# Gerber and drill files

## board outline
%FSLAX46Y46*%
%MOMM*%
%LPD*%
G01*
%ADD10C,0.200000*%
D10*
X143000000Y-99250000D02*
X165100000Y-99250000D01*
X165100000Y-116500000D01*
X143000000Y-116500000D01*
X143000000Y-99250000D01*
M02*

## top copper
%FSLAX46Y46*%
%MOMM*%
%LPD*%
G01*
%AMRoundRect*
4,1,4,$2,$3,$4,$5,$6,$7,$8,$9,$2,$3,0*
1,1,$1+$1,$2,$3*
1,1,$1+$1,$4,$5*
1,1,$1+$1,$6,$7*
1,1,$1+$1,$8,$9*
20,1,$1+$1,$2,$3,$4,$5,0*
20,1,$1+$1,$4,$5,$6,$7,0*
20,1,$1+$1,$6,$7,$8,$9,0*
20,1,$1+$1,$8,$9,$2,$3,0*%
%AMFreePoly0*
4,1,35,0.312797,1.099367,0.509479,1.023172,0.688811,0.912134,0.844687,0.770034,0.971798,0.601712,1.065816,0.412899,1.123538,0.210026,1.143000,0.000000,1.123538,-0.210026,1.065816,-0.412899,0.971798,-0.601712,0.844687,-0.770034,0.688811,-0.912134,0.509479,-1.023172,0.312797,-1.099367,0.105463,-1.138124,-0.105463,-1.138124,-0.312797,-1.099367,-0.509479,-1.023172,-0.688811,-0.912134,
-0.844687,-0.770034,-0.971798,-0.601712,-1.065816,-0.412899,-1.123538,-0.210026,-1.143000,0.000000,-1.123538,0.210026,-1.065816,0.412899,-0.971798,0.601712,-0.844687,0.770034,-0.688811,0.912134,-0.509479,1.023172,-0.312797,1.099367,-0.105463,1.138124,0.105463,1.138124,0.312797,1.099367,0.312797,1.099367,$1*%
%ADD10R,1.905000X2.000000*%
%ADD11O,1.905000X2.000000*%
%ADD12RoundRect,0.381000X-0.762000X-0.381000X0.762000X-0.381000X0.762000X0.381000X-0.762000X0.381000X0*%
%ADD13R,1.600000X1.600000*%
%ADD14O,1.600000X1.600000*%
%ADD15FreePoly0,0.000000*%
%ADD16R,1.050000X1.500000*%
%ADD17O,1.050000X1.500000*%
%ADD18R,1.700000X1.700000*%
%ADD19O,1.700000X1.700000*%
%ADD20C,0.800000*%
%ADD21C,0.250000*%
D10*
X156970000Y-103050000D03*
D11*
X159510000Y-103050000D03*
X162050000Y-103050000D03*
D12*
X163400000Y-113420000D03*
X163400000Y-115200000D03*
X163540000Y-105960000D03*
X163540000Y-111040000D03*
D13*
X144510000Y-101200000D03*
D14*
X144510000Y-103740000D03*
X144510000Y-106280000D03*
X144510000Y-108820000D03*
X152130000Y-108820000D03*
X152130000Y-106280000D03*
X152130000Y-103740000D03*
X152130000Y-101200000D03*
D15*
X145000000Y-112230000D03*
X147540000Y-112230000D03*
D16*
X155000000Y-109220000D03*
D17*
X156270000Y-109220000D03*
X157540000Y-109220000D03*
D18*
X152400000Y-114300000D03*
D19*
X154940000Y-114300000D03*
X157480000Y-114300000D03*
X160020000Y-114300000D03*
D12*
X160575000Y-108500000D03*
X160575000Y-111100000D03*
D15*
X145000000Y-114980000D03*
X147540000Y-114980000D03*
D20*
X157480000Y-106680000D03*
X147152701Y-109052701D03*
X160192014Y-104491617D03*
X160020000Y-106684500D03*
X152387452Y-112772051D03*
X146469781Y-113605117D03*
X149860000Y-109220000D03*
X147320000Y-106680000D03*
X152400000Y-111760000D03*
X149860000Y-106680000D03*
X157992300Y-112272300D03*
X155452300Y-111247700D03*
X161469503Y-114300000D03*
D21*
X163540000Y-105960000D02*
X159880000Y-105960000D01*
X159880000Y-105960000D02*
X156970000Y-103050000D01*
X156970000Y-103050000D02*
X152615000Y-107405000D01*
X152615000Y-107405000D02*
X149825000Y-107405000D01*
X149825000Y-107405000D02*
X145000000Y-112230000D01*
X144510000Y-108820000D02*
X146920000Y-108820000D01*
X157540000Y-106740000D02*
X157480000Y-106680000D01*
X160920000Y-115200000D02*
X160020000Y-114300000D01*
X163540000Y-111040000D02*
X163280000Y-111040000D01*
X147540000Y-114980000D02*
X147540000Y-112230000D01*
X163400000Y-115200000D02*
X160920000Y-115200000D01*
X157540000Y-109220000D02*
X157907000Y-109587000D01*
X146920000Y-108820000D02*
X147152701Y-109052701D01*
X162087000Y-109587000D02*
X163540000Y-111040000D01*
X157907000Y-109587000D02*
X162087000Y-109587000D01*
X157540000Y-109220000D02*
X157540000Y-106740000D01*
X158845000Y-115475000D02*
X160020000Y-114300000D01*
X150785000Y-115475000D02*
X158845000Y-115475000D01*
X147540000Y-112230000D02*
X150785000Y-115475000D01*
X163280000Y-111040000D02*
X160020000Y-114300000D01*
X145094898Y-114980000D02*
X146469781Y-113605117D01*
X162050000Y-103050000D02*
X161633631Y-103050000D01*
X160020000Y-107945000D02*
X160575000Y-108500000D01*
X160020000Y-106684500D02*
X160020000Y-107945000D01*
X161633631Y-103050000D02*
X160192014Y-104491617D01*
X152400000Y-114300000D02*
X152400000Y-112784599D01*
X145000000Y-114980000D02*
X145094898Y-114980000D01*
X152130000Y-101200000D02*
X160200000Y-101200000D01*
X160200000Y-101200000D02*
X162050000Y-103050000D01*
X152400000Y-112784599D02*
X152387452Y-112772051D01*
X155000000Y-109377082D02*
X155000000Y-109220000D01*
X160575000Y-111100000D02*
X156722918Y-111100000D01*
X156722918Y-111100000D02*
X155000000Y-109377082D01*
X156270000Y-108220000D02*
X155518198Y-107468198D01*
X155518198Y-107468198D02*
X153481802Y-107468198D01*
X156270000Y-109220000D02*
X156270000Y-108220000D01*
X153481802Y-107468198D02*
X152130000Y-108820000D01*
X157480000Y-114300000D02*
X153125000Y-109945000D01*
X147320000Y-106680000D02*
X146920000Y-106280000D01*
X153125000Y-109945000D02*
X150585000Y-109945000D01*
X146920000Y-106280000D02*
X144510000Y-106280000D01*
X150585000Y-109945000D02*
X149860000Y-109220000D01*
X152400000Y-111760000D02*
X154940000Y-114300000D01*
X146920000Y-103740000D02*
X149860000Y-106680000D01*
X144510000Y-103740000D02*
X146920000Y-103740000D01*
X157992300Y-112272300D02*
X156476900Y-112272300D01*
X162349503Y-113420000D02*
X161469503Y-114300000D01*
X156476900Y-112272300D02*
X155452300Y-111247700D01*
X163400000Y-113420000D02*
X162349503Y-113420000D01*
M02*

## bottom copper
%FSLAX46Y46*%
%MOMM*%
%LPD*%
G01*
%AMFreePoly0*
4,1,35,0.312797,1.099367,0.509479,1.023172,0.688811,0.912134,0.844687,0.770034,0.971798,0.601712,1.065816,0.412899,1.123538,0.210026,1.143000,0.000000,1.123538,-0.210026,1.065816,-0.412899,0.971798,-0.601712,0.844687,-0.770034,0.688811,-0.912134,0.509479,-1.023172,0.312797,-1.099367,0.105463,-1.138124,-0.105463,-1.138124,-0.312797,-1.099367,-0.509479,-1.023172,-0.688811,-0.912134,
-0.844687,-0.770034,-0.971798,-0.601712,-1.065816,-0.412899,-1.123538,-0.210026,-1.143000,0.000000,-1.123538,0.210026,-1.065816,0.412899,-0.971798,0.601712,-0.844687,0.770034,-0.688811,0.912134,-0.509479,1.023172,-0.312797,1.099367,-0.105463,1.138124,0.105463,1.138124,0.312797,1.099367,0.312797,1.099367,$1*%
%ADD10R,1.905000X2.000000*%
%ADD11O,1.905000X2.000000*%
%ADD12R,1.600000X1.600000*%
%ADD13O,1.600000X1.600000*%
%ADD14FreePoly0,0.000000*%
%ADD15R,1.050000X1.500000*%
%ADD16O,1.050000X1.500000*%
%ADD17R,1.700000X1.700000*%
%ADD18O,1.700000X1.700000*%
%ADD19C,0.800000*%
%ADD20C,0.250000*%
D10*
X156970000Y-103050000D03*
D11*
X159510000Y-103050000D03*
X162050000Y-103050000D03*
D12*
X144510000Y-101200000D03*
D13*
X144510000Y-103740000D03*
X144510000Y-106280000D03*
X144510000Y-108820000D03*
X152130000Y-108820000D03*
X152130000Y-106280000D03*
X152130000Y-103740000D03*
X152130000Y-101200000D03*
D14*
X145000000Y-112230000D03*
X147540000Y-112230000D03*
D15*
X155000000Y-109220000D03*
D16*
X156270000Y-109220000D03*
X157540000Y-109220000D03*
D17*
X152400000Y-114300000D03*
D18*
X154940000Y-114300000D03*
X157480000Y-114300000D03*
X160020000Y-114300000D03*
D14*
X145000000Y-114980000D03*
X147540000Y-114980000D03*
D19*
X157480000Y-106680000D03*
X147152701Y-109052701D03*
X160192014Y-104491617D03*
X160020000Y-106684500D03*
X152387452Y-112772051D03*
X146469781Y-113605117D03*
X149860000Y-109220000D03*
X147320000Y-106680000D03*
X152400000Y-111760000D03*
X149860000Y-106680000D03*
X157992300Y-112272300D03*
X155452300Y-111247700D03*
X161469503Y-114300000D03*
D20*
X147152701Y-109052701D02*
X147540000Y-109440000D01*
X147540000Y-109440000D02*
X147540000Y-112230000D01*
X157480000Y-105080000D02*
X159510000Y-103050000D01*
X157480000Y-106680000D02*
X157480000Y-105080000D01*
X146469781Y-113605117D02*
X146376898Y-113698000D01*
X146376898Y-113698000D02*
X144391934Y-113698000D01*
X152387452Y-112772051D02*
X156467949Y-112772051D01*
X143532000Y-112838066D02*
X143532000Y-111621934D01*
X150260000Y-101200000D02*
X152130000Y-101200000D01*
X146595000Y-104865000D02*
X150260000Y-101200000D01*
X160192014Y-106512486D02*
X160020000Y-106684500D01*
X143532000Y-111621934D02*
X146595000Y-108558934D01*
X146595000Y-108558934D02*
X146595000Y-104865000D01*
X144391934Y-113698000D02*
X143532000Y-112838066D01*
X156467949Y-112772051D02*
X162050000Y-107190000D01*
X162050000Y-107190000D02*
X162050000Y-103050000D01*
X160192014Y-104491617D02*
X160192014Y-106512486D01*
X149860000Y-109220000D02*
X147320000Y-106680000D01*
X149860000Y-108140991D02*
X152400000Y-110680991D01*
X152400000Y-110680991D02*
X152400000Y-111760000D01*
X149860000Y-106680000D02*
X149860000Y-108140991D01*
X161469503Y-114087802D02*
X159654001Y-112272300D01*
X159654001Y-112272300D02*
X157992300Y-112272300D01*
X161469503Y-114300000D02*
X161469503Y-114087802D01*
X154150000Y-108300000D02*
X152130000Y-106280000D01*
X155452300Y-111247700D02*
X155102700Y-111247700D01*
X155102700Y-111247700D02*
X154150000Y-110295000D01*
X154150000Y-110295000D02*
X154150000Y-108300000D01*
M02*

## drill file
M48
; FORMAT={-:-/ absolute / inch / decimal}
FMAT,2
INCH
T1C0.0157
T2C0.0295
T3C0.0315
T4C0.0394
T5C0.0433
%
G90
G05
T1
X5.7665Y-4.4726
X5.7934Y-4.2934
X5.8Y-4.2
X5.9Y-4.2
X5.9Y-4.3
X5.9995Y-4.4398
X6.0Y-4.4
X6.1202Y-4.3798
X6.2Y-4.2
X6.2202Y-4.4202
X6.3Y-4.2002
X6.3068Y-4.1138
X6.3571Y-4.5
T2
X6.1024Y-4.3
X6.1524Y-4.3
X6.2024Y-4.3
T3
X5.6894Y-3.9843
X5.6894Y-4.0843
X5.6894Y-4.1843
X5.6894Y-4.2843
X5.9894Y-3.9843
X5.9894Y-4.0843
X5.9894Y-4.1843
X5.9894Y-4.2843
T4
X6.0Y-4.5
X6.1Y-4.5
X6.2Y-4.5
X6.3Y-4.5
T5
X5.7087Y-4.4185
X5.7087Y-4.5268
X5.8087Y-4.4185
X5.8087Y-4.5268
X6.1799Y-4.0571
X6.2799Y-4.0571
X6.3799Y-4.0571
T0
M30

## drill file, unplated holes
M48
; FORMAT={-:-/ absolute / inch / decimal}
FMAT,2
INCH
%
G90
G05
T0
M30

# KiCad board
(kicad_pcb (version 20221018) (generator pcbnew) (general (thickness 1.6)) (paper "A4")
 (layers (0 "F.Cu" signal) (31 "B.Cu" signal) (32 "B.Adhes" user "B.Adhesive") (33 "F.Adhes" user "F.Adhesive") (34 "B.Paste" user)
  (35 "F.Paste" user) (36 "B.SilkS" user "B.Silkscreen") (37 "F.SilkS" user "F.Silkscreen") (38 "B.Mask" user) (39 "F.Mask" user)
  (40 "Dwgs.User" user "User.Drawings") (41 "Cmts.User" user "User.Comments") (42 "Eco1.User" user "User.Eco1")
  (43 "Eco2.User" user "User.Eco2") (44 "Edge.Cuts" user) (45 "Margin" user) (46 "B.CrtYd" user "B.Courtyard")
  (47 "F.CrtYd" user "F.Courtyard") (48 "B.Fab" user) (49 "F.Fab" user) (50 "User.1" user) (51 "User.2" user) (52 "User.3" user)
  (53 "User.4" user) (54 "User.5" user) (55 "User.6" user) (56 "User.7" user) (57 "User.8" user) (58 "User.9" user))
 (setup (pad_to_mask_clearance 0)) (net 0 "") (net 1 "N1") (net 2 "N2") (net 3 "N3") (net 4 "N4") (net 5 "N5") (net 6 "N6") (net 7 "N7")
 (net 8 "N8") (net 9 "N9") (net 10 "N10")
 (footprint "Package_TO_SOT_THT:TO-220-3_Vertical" (layer "F.Cu") (at 156.97 103.05)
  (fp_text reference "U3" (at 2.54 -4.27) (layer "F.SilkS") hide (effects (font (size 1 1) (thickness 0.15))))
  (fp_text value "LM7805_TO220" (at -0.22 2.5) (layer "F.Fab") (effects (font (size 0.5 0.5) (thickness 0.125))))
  (pad "1" thru_hole rect (at 0 0) (size 1.905 2) (drill 1.1) (layers "*.Cu" "*.Mask") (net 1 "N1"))
  (pad "2" thru_hole oval (at 2.54 0) (size 1.905 2) (drill 1.1) (layers "*.Cu" "*.Mask") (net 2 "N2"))
  (pad "3" thru_hole oval (at 5.08 0) (size 1.905 2) (drill 1.1) (layers "*.Cu" "*.Mask") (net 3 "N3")))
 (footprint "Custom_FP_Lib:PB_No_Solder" (layer "F.Cu") (at 163.4 118.5)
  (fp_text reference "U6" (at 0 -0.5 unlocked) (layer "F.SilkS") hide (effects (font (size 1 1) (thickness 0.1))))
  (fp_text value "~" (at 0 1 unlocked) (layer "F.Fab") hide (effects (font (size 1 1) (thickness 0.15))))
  (pad "1" smd roundrect (at 0 -5.08) (size 2.286 1.524) (layers "F.Cu" "F.Paste" "F.Mask") (roundrect_rratio 0.25) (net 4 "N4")
   (thermal_bridge_angle 45))
  (pad "2" smd roundrect (at 0 -3.3) (size 2.286 1.524) (layers "F.Cu" "F.Paste" "F.Mask") (roundrect_rratio 0.25) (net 2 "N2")
   (thermal_bridge_angle 45)))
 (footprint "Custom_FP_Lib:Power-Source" (layer "F.Cu") (at 161 108.5)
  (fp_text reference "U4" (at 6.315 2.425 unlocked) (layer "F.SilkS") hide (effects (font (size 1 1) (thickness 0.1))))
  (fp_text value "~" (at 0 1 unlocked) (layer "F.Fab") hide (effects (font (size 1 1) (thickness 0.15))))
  (pad "1" smd roundrect (at 2.54 -2.54) (size 2.286 1.524) (layers "F.Cu" "F.Paste" "F.Mask") (roundrect_rratio 0.25) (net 1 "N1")
   (thermal_bridge_angle 45))
  (pad "2" smd roundrect (at 2.54 2.54) (size 2.286 1.524) (layers "F.Cu" "F.Paste" "F.Mask") (roundrect_rratio 0.25) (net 2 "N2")
   (thermal_bridge_angle 45)))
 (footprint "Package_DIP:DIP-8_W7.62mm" (layer "F.Cu") (at 144.51 101.2)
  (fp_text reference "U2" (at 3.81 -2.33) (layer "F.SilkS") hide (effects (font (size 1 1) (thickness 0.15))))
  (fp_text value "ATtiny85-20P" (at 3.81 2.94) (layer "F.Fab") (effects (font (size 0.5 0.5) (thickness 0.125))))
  (pad "1" thru_hole rect (at 0 0) (size 1.6 1.6) (drill 0.8) (layers "*.Cu" "*.Mask") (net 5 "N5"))
  (pad "2" thru_hole oval (at 0 2.54) (size 1.6 1.6) (drill 0.8) (layers "*.Cu" "*.Mask") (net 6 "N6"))
  (pad "3" thru_hole oval (at 0 5.08) (size 1.6 1.6) (drill 0.8) (layers "*.Cu" "*.Mask") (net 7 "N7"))
  (pad "4" thru_hole oval (at 0 7.62) (size 1.6 1.6) (drill 0.8) (layers "*.Cu" "*.Mask") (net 2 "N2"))
  (pad "5" thru_hole oval (at 7.62 7.62) (size 1.6 1.6) (drill 0.8) (layers "*.Cu" "*.Mask") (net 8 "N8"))
  (pad "6" thru_hole oval (at 7.62 5.08) (size 1.6 1.6) (drill 0.8) (layers "*.Cu" "*.Mask") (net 4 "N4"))
  (pad "7" thru_hole oval (at 7.62 2.54) (size 1.6 1.6) (drill 0.8) (layers "*.Cu" "*.Mask") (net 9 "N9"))
  (pad "8" thru_hole oval (at 7.62 0) (size 1.6 1.6) (drill 0.8) (layers "*.Cu" "*.Mask") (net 3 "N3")))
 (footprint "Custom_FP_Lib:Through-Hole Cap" (layer "F.Cu") (at 145 113.5)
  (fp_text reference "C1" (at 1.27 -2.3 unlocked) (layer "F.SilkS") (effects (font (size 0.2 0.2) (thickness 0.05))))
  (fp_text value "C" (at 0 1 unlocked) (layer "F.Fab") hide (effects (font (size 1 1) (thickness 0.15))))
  (pad "1" thru_hole custom (at 0 -1.27) (size 2.286 2.286) (drill 1.1) (layers "*.Cu" "*.Mask") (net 1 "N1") (thermal_bridge_angle 45)
   (options (clearance outline) (anchor circle)) (primitives))
  (pad "2" thru_hole custom (at 2.54 -1.27) (size 2.286 2.286) (drill 1.1) (layers "*.Cu" "*.Mask") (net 2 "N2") (thermal_bridge_angle 45)
   (options (clearance outline) (anchor circle)) (primitives)))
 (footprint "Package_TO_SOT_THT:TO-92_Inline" (layer "F.Cu") (at 155 109.22)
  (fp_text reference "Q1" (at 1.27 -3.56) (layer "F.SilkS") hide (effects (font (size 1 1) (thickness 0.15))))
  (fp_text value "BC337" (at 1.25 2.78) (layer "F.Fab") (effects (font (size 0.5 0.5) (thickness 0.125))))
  (pad "1" thru_hole rect (at 0 0) (size 1.05 1.5) (drill 0.75) (layers "*.Cu" "*.Mask") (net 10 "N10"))
  (pad "2" thru_hole oval (at 1.27 0) (size 1.05 1.5) (drill 0.75) (layers "*.Cu" "*.Mask") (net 8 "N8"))
  (pad "3" thru_hole oval (at 2.54 0) (size 1.05 1.5) (drill 0.75) (layers "*.Cu" "*.Mask") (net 2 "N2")))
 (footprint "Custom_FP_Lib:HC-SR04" (layer "F.Cu") (at 156.32 112.8 90)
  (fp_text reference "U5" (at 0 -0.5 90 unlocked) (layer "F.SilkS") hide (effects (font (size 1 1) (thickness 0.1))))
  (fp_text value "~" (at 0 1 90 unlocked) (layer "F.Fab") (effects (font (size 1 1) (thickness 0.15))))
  (pad "1" thru_hole rect (at -1.5 -3.92 90) (size 1.7 1.7) (drill 1) (layers "*.Cu" "*.Mask") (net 3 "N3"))
  (pad "2" thru_hole oval (at -1.5 -1.38 90) (size 1.7 1.7) (drill 1) (layers "*.Cu" "*.Mask") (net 6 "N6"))
  (pad "3" thru_hole oval (at -1.5 1.16 90) (size 1.7 1.7) (drill 1) (layers "*.Cu" "*.Mask") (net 7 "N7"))
  (pad "4" thru_hole oval (at -1.5 3.7 90) (size 1.7 1.7) (drill 1) (layers "*.Cu" "*.Mask") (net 2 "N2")))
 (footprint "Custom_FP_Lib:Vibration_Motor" (layer "F.Cu") (at 160.575 111.1)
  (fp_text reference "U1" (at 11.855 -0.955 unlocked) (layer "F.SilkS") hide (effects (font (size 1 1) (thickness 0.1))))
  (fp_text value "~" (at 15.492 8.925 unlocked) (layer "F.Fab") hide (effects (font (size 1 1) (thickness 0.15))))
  (pad "1" smd roundrect (at 0 -2.6) (size 2.286 1.524) (layers "F.Cu" "F.Paste" "F.Mask") (roundrect_rratio 0.25) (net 3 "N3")
   (thermal_bridge_angle 45))
  (pad "2" smd roundrect (at 0 0) (size 2.286 1.524) (layers "F.Cu" "F.Paste" "F.Mask") (roundrect_rratio 0.25) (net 10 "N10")
   (thermal_bridge_angle 45)))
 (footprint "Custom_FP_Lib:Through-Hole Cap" (layer "F.Cu") (at 145 116.25)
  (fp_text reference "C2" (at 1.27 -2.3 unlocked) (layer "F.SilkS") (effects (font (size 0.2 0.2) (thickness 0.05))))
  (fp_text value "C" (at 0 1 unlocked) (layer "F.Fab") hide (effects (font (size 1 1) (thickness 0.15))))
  (pad "1" thru_hole custom (at 0 -1.27) (size 2.286 2.286) (drill 1.1) (layers "*.Cu" "*.Mask") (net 3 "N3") (thermal_bridge_angle 45)
   (options (clearance outline) (anchor circle)) (primitives))
  (pad "2" thru_hole custom (at 2.54 -1.27) (size 2.286 2.286) (drill 1.1) (layers "*.Cu" "*.Mask") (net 2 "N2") (thermal_bridge_angle 45)
   (options (clearance outline) (anchor circle)) (primitives)))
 (gr_rect (start 143 99.25) (end 165.1 116.5) (stroke (width 0.2) (type default)) (fill none) (layer "Edge.Cuts"))
 (segment (start 163.54 105.96) (end 159.88 105.96) (width 0.25) (layer "F.Cu") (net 1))
 (segment (start 159.88 105.96) (end 156.97 103.05) (width 0.25) (layer "F.Cu") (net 1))
 (segment (start 156.97 103.05) (end 152.615 107.405) (width 0.25) (layer "F.Cu") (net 1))
 (segment (start 152.615 107.405) (end 149.825 107.405) (width 0.25) (layer "F.Cu") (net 1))
 (segment (start 149.825 107.405) (end 145 112.23) (width 0.25) (layer "F.Cu") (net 1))
 (segment (start 144.51 108.82) (end 146.92 108.82) (width 0.25) (layer "F.Cu") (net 2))
 (segment (start 157.54 106.74) (end 157.48 106.68) (width 0.25) (layer "F.Cu") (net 2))
 (segment (start 160.92 115.2) (end 160.02 114.3) (width 0.25) (layer "F.Cu") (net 2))
 (segment (start 163.54 111.04) (end 163.28 111.04) (width 0.25) (layer "F.Cu") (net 2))
 (segment (start 147.54 114.98) (end 147.54 112.23) (width 0.25) (layer "F.Cu") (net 2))
 (segment (start 163.4 115.2) (end 160.92 115.2) (width 0.25) (layer "F.Cu") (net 2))
 (segment (start 157.54 109.22) (end 157.907 109.587) (width 0.25) (layer "F.Cu") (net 2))
 (segment (start 146.92 108.82) (end 147.152701 109.052701) (width 0.25) (layer "F.Cu") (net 2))
 (segment (start 162.087 109.587) (end 163.54 111.04) (width 0.25) (layer "F.Cu") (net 2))
 (segment (start 157.907 109.587) (end 162.087 109.587) (width 0.25) (layer "F.Cu") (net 2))
 (segment (start 157.54 109.22) (end 157.54 106.74) (width 0.25) (layer "F.Cu") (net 2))
 (segment (start 158.845 115.475) (end 160.02 114.3) (width 0.25) (layer "F.Cu") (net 2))
 (segment (start 150.785 115.475) (end 158.845 115.475) (width 0.25) (layer "F.Cu") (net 2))
 (segment (start 147.54 112.23) (end 150.785 115.475) (width 0.25) (layer "F.Cu") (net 2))
 (segment (start 163.28 111.04) (end 160.02 114.3) (width 0.25) (layer "F.Cu") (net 2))
 (via (at 157.48 106.68) (size 0.8) (drill 0.4) (layers "F.Cu" "B.Cu") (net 2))
 (via (at 147.152701 109.052701) (size 0.8) (drill 0.4) (layers "F.Cu" "B.Cu") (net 2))
 (segment (start 147.152701 109.052701) (end 147.54 109.44) (width 0.25) (layer "B.Cu") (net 2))
 (segment (start 147.54 109.44) (end 147.54 112.23) (width 0.25) (layer "B.Cu") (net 2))
 (segment (start 157.48 105.08) (end 159.51 103.05) (width 0.25) (layer "B.Cu") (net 2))
 (segment (start 157.48 106.68) (end 157.48 105.08) (width 0.25) (layer "B.Cu") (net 2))
 (segment (start 145.094898 114.98) (end 146.469781 113.605117) (width 0.25) (layer "F.Cu") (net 3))
 (segment (start 162.05 103.05) (end 161.633631 103.05) (width 0.25) (layer "F.Cu") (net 3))
 (segment (start 160.02 107.945) (end 160.575 108.5) (width 0.25) (layer "F.Cu") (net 3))
 (segment (start 160.02 106.6845) (end 160.02 107.945) (width 0.25) (layer "F.Cu") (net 3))
 (segment (start 161.633631 103.05) (end 160.192014 104.491617) (width 0.25) (layer "F.Cu") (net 3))
 (segment (start 152.4 114.3) (end 152.4 112.784599) (width 0.25) (layer "F.Cu") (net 3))
 (segment (start 145 114.98) (end 145.094898 114.98) (width 0.25) (layer "F.Cu") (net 3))
 (segment (start 152.13 101.2) (end 160.2 101.2) (width 0.25) (layer "F.Cu") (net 3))
 (segment (start 160.2 101.2) (end 162.05 103.05) (width 0.25) (layer "F.Cu") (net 3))
 (segment (start 152.4 112.784599) (end 152.387452 112.772051) (width 0.25) (layer "F.Cu") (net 3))
 (via (at 160.192014 104.491617) (size 0.8) (drill 0.4) (layers "F.Cu" "B.Cu") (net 3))
 (via (at 160.02 106.6845) (size 0.8) (drill 0.4) (layers "F.Cu" "B.Cu") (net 3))
 (via (at 152.387452 112.772051) (size 0.8) (drill 0.4) (layers "F.Cu" "B.Cu") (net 3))
 (via (at 146.469781 113.605117) (size 0.8) (drill 0.4) (layers "F.Cu" "B.Cu") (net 3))
 (segment (start 146.469781 113.605117) (end 146.376898 113.698) (width 0.25) (layer "B.Cu") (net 3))
 (segment (start 146.376898 113.698) (end 144.391934 113.698) (width 0.25) (layer "B.Cu") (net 3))
 (segment (start 152.387452 112.772051) (end 156.467949 112.772051) (width 0.25) (layer "B.Cu") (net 3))
 (segment (start 143.532 112.838066) (end 143.532 111.621934) (width 0.25) (layer "B.Cu") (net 3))
 (segment (start 150.26 101.2) (end 152.13 101.2) (width 0.25) (layer "B.Cu") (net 3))
 (segment (start 146.595 104.865) (end 150.26 101.2) (width 0.25) (layer "B.Cu") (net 3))
 (segment (start 160.192014 106.512486) (end 160.02 106.6845) (width 0.25) (layer "B.Cu") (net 3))
 (segment (start 143.532 111.621934) (end 146.595 108.558934) (width 0.25) (layer "B.Cu") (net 3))
 (segment (start 146.595 108.558934) (end 146.595 104.865) (width 0.25) (layer "B.Cu") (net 3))
 (segment (start 144.391934 113.698) (end 143.532 112.838066) (width 0.25) (layer "B.Cu") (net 3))
 (segment (start 156.467949 112.772051) (end 162.05 107.19) (width 0.25) (layer "B.Cu") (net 3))
 (segment (start 162.05 107.19) (end 162.05 103.05) (width 0.25) (layer "B.Cu") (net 3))
 (segment (start 160.192014 104.491617) (end 160.192014 106.512486) (width 0.25) (layer "B.Cu") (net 3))
 (segment (start 155 109.377082) (end 155 109.22) (width 0.25) (layer "F.Cu") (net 10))
 (segment (start 160.575 111.1) (end 156.722918 111.1) (width 0.25) (layer "F.Cu") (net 10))
 (segment (start 156.722918 111.1) (end 155 109.377082) (width 0.25) (layer "F.Cu") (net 10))
 (segment (start 156.27 108.22) (end 155.518198 107.468198) (width 0.25) (layer "F.Cu") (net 8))
 (segment (start 155.518198 107.468198) (end 153.481802 107.468198) (width 0.25) (layer "F.Cu") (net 8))
 (segment (start 156.27 109.22) (end 156.27 108.22) (width 0.25) (layer "F.Cu") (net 8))
 (segment (start 153.481802 107.468198) (end 152.13 108.82) (width 0.25) (layer "F.Cu") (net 8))
 (segment (start 157.48 114.3) (end 153.125 109.945) (width 0.25) (layer "F.Cu") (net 7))
 (segment (start 147.32 106.68) (end 146.92 106.28) (width 0.25) (layer "F.Cu") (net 7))
 (segment (start 153.125 109.945) (end 150.585 109.945) (width 0.25) (layer "F.Cu") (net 7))
 (segment (start 146.92 106.28) (end 144.51 106.28) (width 0.25) (layer "F.Cu") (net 7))
 (segment (start 150.585 109.945) (end 149.86 109.22) (width 0.25) (layer "F.Cu") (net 7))
 (via (at 149.86 109.22) (size 0.8) (drill 0.4) (layers "F.Cu" "B.Cu") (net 7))
 (via (at 147.32 106.68) (size 0.8) (drill 0.4) (layers "F.Cu" "B.Cu") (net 7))
 (segment (start 149.86 109.22) (end 147.32 106.68) (width 0.25) (layer "B.Cu") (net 7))
 (segment (start 152.4 111.76) (end 154.94 114.3) (width 0.25) (layer "F.Cu") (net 6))
 (segment (start 146.92 103.74) (end 149.86 106.68) (width 0.25) (layer "F.Cu") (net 6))
 (segment (start 144.51 103.74) (end 146.92 103.74) (width 0.25) (layer "F.Cu") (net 6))
 (via (at 152.4 111.76) (size 0.8) (drill 0.4) (layers "F.Cu" "B.Cu") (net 6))
 (via (at 149.86 106.68) (size 0.8) (drill 0.4) (layers "F.Cu" "B.Cu") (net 6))
 (segment (start 149.86 108.140991) (end 152.4 110.680991) (width 0.25) (layer "B.Cu") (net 6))
 (segment (start 152.4 110.680991) (end 152.4 111.76) (width 0.25) (layer "B.Cu") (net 6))
 (segment (start 149.86 106.68) (end 149.86 108.140991) (width 0.25) (layer "B.Cu") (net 6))
 (segment (start 157.9923 112.2723) (end 156.4769 112.2723) (width 0.25) (layer "F.Cu") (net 4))
 (segment (start 162.349503 113.42) (end 161.469503 114.3) (width 0.25) (layer "F.Cu") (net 4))
 (segment (start 156.4769 112.2723) (end 155.4523 111.2477) (width 0.25) (layer "F.Cu") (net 4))
 (segment (start 163.4 113.42) (end 162.349503 113.42) (width 0.25) (layer "F.Cu") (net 4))
 (via (at 157.9923 112.2723) (size 0.8) (drill 0.4) (layers "F.Cu" "B.Cu") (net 4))
 (via (at 155.4523 111.2477) (size 0.8) (drill 0.4) (layers "F.Cu" "B.Cu") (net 4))
 (via (at 161.469503 114.3) (size 0.8) (drill 0.4) (layers "F.Cu" "B.Cu") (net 4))
 (segment (start 161.469503 114.087802) (end 159.654001 112.2723) (width 0.25) (layer "B.Cu") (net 4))
 (segment (start 159.654001 112.2723) (end 157.9923 112.2723) (width 0.25) (layer "B.Cu") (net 4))
 (segment (start 161.469503 114.3) (end 161.469503 114.087802) (width 0.25) (layer "B.Cu") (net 4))
 (segment (start 154.15 108.3) (end 152.13 106.28) (width 0.25) (layer "B.Cu") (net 4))
 (segment (start 155.4523 111.2477) (end 155.1027 111.2477) (width 0.25) (layer "B.Cu") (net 4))
 (segment (start 155.1027 111.2477) (end 154.15 110.295) (width 0.25) (layer "B.Cu") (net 4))
 (segment (start 154.15 110.295) (end 154.15 108.3) (width 0.25) (layer "B.Cu") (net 4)))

